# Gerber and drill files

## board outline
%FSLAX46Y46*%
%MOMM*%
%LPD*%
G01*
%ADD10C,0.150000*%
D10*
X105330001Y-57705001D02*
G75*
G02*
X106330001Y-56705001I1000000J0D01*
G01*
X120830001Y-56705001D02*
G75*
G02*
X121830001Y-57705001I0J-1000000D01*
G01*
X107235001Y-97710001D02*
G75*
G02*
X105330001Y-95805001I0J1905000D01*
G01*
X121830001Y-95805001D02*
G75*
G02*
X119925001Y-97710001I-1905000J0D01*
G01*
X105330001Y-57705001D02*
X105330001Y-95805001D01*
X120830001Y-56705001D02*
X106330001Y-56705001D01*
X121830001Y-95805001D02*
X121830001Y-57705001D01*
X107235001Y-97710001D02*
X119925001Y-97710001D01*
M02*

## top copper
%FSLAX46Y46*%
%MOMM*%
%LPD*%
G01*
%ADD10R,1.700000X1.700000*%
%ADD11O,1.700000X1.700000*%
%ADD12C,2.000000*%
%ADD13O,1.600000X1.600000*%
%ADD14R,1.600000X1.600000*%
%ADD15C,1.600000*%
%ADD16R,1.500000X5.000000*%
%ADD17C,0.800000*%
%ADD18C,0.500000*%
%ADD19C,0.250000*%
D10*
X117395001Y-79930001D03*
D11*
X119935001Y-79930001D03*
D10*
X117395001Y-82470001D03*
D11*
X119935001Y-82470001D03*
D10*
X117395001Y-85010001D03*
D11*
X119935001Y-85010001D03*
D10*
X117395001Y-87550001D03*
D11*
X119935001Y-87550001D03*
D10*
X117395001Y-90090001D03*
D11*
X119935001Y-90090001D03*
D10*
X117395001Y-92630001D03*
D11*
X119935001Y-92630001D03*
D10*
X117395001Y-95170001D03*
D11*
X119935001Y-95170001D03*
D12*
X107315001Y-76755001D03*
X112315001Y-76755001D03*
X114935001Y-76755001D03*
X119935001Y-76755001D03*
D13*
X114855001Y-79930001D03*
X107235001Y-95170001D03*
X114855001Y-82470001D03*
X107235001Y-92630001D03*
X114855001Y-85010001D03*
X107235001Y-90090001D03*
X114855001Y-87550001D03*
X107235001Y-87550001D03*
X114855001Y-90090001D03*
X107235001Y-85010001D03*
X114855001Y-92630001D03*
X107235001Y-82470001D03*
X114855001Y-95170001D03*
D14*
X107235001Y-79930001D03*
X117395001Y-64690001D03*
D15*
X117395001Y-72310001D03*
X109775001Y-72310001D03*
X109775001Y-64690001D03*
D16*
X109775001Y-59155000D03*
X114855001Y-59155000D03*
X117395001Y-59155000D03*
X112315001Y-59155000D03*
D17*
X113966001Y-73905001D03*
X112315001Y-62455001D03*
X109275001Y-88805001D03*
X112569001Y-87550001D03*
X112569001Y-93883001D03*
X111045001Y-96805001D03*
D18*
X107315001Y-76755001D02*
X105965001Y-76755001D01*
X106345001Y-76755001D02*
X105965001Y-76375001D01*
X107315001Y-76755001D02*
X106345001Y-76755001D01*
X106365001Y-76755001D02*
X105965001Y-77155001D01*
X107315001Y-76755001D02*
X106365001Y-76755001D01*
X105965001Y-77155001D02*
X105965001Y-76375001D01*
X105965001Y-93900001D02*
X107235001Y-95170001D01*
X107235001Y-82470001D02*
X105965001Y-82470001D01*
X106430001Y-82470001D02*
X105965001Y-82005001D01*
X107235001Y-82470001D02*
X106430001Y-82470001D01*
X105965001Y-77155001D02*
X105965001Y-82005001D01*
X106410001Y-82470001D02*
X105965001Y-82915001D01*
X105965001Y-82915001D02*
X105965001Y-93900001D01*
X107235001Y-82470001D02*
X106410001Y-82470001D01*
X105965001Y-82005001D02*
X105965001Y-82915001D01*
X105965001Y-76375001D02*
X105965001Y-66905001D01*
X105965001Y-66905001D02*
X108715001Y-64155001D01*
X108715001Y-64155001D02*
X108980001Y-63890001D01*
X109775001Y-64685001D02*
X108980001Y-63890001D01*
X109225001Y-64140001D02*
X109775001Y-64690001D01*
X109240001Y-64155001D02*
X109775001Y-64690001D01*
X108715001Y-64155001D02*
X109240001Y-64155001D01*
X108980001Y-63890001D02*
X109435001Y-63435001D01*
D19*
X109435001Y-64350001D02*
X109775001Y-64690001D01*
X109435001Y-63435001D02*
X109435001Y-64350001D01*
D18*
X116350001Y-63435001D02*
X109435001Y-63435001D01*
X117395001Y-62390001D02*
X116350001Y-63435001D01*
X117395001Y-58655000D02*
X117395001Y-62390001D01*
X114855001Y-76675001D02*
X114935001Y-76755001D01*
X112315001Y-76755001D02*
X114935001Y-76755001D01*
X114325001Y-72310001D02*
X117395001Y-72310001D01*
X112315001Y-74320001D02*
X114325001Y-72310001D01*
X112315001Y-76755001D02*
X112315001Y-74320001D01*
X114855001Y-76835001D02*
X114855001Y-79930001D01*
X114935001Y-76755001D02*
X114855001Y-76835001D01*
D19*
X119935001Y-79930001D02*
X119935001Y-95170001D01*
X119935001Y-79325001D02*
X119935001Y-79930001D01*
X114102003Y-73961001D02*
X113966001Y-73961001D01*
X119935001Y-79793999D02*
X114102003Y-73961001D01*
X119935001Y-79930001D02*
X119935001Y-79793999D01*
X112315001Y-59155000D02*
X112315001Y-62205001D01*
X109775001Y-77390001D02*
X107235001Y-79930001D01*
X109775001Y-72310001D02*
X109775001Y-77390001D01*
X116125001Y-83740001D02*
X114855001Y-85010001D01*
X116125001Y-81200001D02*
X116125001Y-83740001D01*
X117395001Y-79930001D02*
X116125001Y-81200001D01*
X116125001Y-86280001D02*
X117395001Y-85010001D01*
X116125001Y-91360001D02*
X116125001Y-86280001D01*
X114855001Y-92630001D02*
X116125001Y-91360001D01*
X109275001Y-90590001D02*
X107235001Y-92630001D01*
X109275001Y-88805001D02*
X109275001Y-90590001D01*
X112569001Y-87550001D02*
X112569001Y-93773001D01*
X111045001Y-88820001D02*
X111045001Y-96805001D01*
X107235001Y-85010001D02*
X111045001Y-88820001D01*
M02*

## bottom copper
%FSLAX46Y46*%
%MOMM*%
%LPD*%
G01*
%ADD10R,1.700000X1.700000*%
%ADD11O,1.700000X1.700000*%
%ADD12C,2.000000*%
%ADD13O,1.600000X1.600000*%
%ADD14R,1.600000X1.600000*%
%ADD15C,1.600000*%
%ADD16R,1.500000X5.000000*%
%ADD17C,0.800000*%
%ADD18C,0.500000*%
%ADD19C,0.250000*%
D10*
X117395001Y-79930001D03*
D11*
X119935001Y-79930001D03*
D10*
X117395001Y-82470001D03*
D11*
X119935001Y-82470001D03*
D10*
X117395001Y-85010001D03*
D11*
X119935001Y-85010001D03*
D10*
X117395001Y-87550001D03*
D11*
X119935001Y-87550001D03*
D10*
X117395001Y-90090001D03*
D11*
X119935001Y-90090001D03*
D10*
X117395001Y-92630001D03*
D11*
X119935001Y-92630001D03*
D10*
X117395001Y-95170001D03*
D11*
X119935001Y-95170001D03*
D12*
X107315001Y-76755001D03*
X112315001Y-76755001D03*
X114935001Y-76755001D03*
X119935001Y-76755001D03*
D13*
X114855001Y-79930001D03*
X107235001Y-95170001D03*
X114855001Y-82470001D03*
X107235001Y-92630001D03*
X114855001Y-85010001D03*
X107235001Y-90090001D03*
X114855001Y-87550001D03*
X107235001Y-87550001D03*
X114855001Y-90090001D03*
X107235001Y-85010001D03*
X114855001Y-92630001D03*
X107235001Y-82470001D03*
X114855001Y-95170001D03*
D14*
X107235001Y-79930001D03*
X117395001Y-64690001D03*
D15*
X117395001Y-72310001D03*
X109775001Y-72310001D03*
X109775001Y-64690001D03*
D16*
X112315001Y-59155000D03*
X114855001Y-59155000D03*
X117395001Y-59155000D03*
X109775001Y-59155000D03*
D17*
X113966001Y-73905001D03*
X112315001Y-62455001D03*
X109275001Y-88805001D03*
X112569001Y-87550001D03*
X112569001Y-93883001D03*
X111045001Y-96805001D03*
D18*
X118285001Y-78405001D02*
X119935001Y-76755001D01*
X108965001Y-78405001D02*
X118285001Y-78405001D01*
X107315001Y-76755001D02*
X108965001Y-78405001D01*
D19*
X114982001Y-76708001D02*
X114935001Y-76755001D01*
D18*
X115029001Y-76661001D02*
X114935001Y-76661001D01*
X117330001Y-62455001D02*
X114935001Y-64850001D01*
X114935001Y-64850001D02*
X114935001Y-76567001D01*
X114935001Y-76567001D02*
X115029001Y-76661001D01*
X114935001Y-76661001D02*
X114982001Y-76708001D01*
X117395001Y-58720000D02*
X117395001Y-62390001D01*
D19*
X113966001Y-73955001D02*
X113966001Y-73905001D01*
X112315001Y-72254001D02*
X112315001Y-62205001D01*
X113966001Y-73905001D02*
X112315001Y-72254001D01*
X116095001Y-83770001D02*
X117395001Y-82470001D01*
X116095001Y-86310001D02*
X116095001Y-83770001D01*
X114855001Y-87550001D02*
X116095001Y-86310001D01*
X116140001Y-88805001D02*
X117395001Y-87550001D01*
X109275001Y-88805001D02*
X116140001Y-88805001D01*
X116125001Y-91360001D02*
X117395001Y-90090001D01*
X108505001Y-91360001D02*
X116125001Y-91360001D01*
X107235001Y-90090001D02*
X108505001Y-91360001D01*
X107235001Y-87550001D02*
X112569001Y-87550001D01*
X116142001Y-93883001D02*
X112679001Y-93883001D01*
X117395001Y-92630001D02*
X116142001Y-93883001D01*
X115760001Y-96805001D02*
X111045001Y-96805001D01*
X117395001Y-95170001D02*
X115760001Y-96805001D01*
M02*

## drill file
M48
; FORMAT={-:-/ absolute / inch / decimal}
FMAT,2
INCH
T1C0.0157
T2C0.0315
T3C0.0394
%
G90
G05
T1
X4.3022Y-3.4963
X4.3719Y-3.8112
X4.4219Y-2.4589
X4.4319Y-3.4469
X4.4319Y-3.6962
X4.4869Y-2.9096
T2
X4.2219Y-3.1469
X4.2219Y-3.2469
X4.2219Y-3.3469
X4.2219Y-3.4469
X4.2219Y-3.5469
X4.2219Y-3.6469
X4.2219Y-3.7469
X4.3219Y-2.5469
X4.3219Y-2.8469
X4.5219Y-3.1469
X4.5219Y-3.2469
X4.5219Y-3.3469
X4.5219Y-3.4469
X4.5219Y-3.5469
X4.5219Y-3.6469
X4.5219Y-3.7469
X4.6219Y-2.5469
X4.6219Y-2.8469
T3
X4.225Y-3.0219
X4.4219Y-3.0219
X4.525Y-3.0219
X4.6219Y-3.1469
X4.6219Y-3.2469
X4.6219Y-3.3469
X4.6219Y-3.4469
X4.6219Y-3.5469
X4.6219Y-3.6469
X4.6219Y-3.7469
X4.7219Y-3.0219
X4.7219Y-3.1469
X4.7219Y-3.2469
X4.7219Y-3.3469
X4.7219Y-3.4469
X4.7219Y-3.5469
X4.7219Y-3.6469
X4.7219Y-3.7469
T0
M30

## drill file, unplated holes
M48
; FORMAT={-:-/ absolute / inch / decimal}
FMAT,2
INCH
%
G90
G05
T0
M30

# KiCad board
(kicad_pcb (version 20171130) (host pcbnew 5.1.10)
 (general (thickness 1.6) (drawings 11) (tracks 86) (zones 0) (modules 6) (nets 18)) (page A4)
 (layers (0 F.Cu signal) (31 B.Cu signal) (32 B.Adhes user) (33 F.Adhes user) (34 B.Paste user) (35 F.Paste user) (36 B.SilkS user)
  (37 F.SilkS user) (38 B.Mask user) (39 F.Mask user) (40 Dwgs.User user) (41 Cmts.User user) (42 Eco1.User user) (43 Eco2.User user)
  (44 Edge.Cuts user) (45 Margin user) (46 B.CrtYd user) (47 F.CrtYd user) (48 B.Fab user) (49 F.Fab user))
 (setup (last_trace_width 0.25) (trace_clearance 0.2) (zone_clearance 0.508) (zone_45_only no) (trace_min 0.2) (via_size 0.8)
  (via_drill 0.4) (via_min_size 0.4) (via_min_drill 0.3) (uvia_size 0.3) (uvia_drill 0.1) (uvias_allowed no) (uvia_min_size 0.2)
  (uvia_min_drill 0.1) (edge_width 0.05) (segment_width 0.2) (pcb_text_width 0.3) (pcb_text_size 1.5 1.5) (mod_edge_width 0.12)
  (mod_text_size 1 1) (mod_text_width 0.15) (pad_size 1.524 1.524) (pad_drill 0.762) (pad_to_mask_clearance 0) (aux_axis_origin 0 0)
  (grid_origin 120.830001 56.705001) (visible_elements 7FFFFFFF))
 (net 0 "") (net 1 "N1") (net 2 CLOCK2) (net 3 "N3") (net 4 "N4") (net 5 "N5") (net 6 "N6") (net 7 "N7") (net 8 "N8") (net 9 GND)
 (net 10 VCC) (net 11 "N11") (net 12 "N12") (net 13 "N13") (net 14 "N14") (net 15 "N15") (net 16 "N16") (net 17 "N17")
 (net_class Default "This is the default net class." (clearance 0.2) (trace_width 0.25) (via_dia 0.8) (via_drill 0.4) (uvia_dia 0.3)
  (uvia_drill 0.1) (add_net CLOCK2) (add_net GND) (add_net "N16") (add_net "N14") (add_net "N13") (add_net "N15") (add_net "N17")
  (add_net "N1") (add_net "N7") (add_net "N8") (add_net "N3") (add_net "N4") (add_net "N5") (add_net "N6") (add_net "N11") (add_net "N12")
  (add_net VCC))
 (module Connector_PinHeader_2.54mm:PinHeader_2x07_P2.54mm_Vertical (layer F.Cu) (at 117.395001 79.930001)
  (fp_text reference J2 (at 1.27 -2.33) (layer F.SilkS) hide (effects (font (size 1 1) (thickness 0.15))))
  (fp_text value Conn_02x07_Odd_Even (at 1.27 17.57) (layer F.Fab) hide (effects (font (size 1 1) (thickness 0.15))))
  (pad 1 thru_hole rect (at 0 0) (size 1.7 1.7) (drill 1) (layers *.Cu *.Mask) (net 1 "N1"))
  (pad 2 thru_hole oval (at 2.54 0) (size 1.7 1.7) (drill 1) (layers *.Cu *.Mask) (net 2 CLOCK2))
  (pad 3 thru_hole rect (at 0 2.54) (size 1.7 1.7) (drill 1) (layers *.Cu *.Mask) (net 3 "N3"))
  (pad 4 thru_hole oval (at 2.54 2.54) (size 1.7 1.7) (drill 1) (layers *.Cu *.Mask) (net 2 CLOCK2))
  (pad 5 thru_hole rect (at 0 5.08) (size 1.7 1.7) (drill 1) (layers *.Cu *.Mask) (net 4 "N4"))
  (pad 6 thru_hole oval (at 2.54 5.08) (size 1.7 1.7) (drill 1) (layers *.Cu *.Mask) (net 2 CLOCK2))
  (pad 7 thru_hole rect (at 0 7.62) (size 1.7 1.7) (drill 1) (layers *.Cu *.Mask) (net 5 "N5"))
  (pad 8 thru_hole oval (at 2.54 7.62) (size 1.7 1.7) (drill 1) (layers *.Cu *.Mask) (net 2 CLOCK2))
  (pad 9 thru_hole rect (at 0 10.16) (size 1.7 1.7) (drill 1) (layers *.Cu *.Mask) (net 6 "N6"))
  (pad 10 thru_hole oval (at 2.54 10.16) (size 1.7 1.7) (drill 1) (layers *.Cu *.Mask) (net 2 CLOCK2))
  (pad 11 thru_hole rect (at 0 12.7) (size 1.7 1.7) (drill 1) (layers *.Cu *.Mask) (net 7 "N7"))
  (pad 12 thru_hole oval (at 2.54 12.7) (size 1.7 1.7) (drill 1) (layers *.Cu *.Mask) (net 2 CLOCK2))
  (pad 13 thru_hole rect (at 0 15.24) (size 1.7 1.7) (drill 1) (layers *.Cu *.Mask) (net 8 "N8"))
  (pad 14 thru_hole oval (at 2.54 15.24) (size 1.7 1.7) (drill 1) (layers *.Cu *.Mask) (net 2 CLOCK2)))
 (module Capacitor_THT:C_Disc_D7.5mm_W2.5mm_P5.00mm (layer F.Cu) (at 112.315001 76.755001 180)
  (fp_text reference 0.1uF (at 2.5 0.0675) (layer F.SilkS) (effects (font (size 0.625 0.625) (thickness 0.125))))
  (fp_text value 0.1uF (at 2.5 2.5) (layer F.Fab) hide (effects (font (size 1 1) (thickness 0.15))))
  (pad 2 thru_hole circle (at 5 0 180) (size 2 2) (drill 1) (layers *.Cu *.Mask) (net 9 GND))
  (pad 1 thru_hole circle (at 0 0 180) (size 2 2) (drill 1) (layers *.Cu *.Mask) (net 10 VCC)))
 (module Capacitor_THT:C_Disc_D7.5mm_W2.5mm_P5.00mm (layer F.Cu) (at 114.935001 76.755001)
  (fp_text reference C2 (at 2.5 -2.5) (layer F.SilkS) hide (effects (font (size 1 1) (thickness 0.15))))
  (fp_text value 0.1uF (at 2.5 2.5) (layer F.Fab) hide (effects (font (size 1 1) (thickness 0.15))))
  (pad 1 thru_hole circle (at 0 0) (size 2 2) (drill 1) (layers *.Cu *.Mask) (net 10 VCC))
  (pad 2 thru_hole circle (at 5 0) (size 2 2) (drill 1) (layers *.Cu *.Mask) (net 9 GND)))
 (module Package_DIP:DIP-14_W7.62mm (layer F.Cu) (at 107.235001 79.930001)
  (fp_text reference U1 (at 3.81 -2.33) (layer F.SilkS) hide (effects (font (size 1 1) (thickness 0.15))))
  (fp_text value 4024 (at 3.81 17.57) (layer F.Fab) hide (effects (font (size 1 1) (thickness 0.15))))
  (pad 14 thru_hole oval (at 7.62 0) (size 1.6 1.6) (drill 0.8) (layers *.Cu *.Mask) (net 10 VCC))
  (pad 7 thru_hole oval (at 0 15.24) (size 1.6 1.6) (drill 0.8) (layers *.Cu *.Mask) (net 9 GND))
  (pad 13 thru_hole oval (at 7.62 2.54) (size 1.6 1.6) (drill 0.8) (layers *.Cu *.Mask))
  (pad 6 thru_hole oval (at 0 12.7) (size 1.6 1.6) (drill 0.8) (layers *.Cu *.Mask) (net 5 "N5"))
  (pad 12 thru_hole oval (at 7.62 5.08) (size 1.6 1.6) (drill 0.8) (layers *.Cu *.Mask) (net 1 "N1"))
  (pad 5 thru_hole oval (at 0 10.16) (size 1.6 1.6) (drill 0.8) (layers *.Cu *.Mask) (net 6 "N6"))
  (pad 11 thru_hole oval (at 7.62 7.62) (size 1.6 1.6) (drill 0.8) (layers *.Cu *.Mask) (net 3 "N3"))
  (pad 4 thru_hole oval (at 0 7.62) (size 1.6 1.6) (drill 0.8) (layers *.Cu *.Mask) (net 7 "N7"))
  (pad 10 thru_hole oval (at 7.62 10.16) (size 1.6 1.6) (drill 0.8) (layers *.Cu *.Mask))
  (pad 3 thru_hole oval (at 0 5.08) (size 1.6 1.6) (drill 0.8) (layers *.Cu *.Mask) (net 8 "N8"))
  (pad 9 thru_hole oval (at 7.62 12.7) (size 1.6 1.6) (drill 0.8) (layers *.Cu *.Mask) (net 4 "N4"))
  (pad 2 thru_hole oval (at 0 2.54) (size 1.6 1.6) (drill 0.8) (layers *.Cu *.Mask) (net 9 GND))
  (pad 8 thru_hole oval (at 7.62 15.24) (size 1.6 1.6) (drill 0.8) (layers *.Cu *.Mask))
  (pad 1 thru_hole rect (at 0 0) (size 1.6 1.6) (drill 0.8) (layers *.Cu *.Mask) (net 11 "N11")))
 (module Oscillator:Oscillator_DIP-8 (layer F.Cu) (at 117.395001 64.690001 180)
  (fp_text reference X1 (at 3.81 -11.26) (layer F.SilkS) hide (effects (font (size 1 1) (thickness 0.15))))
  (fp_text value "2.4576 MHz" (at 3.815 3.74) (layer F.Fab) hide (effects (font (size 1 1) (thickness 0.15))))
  (pad 1 thru_hole rect (at 0 0 180) (size 1.6 1.6) (drill 0.8) (layers *.Cu *.Mask) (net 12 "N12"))
  (pad 8 thru_hole circle (at 0 -7.62 180) (size 1.6 1.6) (drill 0.8) (layers *.Cu *.Mask) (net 10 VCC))
  (pad 5 thru_hole circle (at 7.62 -7.62 180) (size 1.6 1.6) (drill 0.8) (layers *.Cu *.Mask) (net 11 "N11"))
  (pad 4 thru_hole circle (at 7.62 0 180) (size 1.6 1.6) (drill 0.8) (layers *.Cu *.Mask) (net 9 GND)))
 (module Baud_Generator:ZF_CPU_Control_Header (layer F.Cu) (at 113.585001 59.028)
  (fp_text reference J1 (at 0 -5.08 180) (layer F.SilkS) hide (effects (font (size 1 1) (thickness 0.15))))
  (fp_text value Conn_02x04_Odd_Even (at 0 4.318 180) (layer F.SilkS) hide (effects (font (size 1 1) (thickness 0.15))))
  (pad 6 connect rect (at -1.27 0.127 180) (size 1.5 5) (layers B.Cu) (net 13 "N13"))
  (pad 4 connect rect (at 1.27 0.127 180) (size 1.5 5) (layers B.Cu) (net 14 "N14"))
  (pad 2 connect rect (at 3.81 0.127 180) (size 1.5 5) (layers B.Cu) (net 10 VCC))
  (pad 7 connect rect (at -3.81 0.127 180) (size 1.5 5) (layers F.Cu) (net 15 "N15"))
  (pad 3 connect rect (at 1.27 0.127 180) (size 1.5 5) (layers F.Cu) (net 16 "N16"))
  (pad 1 connect rect (at 3.81 0.127 180) (size 1.5 5) (layers F.Cu) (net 9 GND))
  (pad 5 connect rect (at -1.27 0.127 180) (size 1.5 5) (layers F.Cu) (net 2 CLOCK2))
  (pad 8 connect rect (at -3.81 0.127 180) (size 1.5 5) (layers B.Cu) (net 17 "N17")))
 (gr_arc (start 106.330001 57.705001) (end 106.330001 56.705001) (angle -90) (layer Edge.Cuts) (width 0.15))
 (gr_arc (start 120.830001 57.705001) (end 121.830001 57.705001) (angle -90) (layer Edge.Cuts) (width 0.15))
 (gr_arc (start 107.235001 95.805001) (end 105.330001 95.805001) (angle -90) (layer Edge.Cuts) (width 0.15))
 (gr_arc (start 119.925001 95.805001) (end 119.925001 97.710001) (angle -90) (layer Edge.Cuts) (width 0.15))
 (gr_line (start 105.330001 57.705001) (end 105.330001 95.805001) (layer Edge.Cuts) (width 0.15))
 (gr_line (start 120.830001 56.705001) (end 106.330001 56.705001) (layer Edge.Cuts) (width 0.15))
 (gr_line (start 121.830001 95.805001) (end 121.830001 57.705001) (layer Edge.Cuts) (width 0.15))
 (gr_line (start 107.235001 97.710001) (end 119.925001 97.710001) (layer Edge.Cuts) (width 0.15))
 (segment (start 107.315001 76.755001) (end 105.965001 76.755001) (width 0.5) (layer F.Cu) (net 9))
 (segment (start 106.345001 76.755001) (end 105.965001 76.375001) (width 0.5) (layer F.Cu) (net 9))
 (segment (start 107.315001 76.755001) (end 106.345001 76.755001) (width 0.5) (layer F.Cu) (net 9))
 (segment (start 106.365001 76.755001) (end 105.965001 77.155001) (width 0.5) (layer F.Cu) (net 9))
 (segment (start 107.315001 76.755001) (end 106.365001 76.755001) (width 0.5) (layer F.Cu) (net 9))
 (segment (start 105.965001 77.155001) (end 105.965001 76.375001) (width 0.5) (layer F.Cu) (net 9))
 (segment (start 105.965001 93.900001) (end 107.235001 95.170001) (width 0.5) (layer F.Cu) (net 9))
 (segment (start 107.235001 82.470001) (end 105.965001 82.470001) (width 0.5) (layer F.Cu) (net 9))
 (segment (start 106.430001 82.470001) (end 105.965001 82.005001) (width 0.5) (layer F.Cu) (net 9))
 (segment (start 107.235001 82.470001) (end 106.430001 82.470001) (width 0.5) (layer F.Cu) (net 9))
 (segment (start 105.965001 77.155001) (end 105.965001 82.005001) (width 0.5) (layer F.Cu) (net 9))
 (segment (start 106.410001 82.470001) (end 105.965001 82.915001) (width 0.5) (layer F.Cu) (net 9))
 (segment (start 105.965001 82.915001) (end 105.965001 93.900001) (width 0.5) (layer F.Cu) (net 9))
 (segment (start 107.235001 82.470001) (end 106.410001 82.470001) (width 0.5) (layer F.Cu) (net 9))
 (segment (start 105.965001 82.005001) (end 105.965001 82.915001) (width 0.5) (layer F.Cu) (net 9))
 (segment (start 105.965001 76.375001) (end 105.965001 66.905001) (width 0.5) (layer F.Cu) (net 9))
 (segment (start 105.965001 66.905001) (end 108.715001 64.155001) (width 0.5) (layer F.Cu) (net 9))
 (segment (start 108.715001 64.155001) (end 108.980001 63.890001) (width 0.5) (layer F.Cu) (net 9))
 (segment (start 109.775001 64.685001) (end 108.980001 63.890001) (width 0.5) (layer F.Cu) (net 9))
 (segment (start 109.225001 64.140001) (end 109.775001 64.690001) (width 0.5) (layer F.Cu) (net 9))
 (segment (start 109.240001 64.155001) (end 109.775001 64.690001) (width 0.5) (layer F.Cu) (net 9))
 (segment (start 108.715001 64.155001) (end 109.240001 64.155001) (width 0.5) (layer F.Cu) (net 9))
 (segment (start 118.285001 78.405001) (end 119.935001 76.755001) (width 0.5) (layer B.Cu) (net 9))
 (segment (start 108.965001 78.405001) (end 118.285001 78.405001) (width 0.5) (layer B.Cu) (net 9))
 (segment (start 107.315001 76.755001) (end 108.965001 78.405001) (width 0.5) (layer B.Cu) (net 9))
 (segment (start 108.980001 63.890001) (end 109.435001 63.435001) (width 0.5) (layer F.Cu) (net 9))
 (segment (start 109.435001 64.350001) (end 109.775001 64.690001) (width 0.25) (layer F.Cu) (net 9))
 (segment (start 109.435001 63.435001) (end 109.435001 64.350001) (width 0.25) (layer F.Cu) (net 9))
 (segment (start 116.350001 63.435001) (end 109.435001 63.435001) (width 0.5) (layer F.Cu) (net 9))
 (segment (start 117.395001 62.390001) (end 116.350001 63.435001) (width 0.5) (layer F.Cu) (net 9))
 (segment (start 117.395001 58.655) (end 117.395001 62.390001) (width 0.5) (layer F.Cu) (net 9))
 (segment (start 114.855001 76.675001) (end 114.935001 76.755001) (width 0.5) (layer F.Cu) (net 10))
 (segment (start 112.315001 76.755001) (end 114.935001 76.755001) (width 0.5) (layer F.Cu) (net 10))
 (segment (start 114.982001 76.708001) (end 114.935001 76.755001) (width 0.25) (layer B.Cu) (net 10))
 (segment (start 114.325001 72.310001) (end 117.395001 72.310001) (width 0.5) (layer F.Cu) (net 10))
 (segment (start 112.315001 74.320001) (end 114.325001 72.310001) (width 0.5) (layer F.Cu) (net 10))
 (segment (start 112.315001 76.755001) (end 112.315001 74.320001) (width 0.5) (layer F.Cu) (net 10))
 (segment (start 114.855001 76.835001) (end 114.855001 79.930001) (width 0.5) (layer F.Cu) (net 10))
 (segment (start 114.935001 76.755001) (end 114.855001 76.835001) (width 0.5) (layer F.Cu) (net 10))
 (segment (start 115.029001 76.661001) (end 114.935001 76.661001) (width 0.5) (layer B.Cu) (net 10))
 (segment (start 117.330001 62.455001) (end 114.935001 64.850001) (width 0.5) (layer B.Cu) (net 10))
 (segment (start 114.935001 64.850001) (end 114.935001 76.567001) (width 0.5) (layer B.Cu) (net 10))
 (segment (start 114.935001 76.567001) (end 115.029001 76.661001) (width 0.5) (layer B.Cu) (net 10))
 (segment (start 114.935001 76.661001) (end 114.982001 76.708001) (width 0.5) (layer B.Cu) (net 10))
 (segment (start 117.395001 58.72) (end 117.395001 62.390001) (width 0.5) (layer B.Cu) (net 10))
 (segment (start 119.935001 79.930001) (end 119.935001 95.170001) (width 0.25) (layer F.Cu) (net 2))
 (segment (start 119.935001 79.325001) (end 119.935001 79.930001) (width 0.25) (layer F.Cu) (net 2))
 (via (at 113.966001 73.905001) (size 0.8) (drill 0.4) (layers F.Cu B.Cu) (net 2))
 (via (at 112.315001 62.455001) (size 0.8) (drill 0.4) (layers F.Cu B.Cu) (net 2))
 (segment (start 114.102003 73.961001) (end 113.966001 73.961001) (width 0.25) (layer F.Cu) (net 2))
 (segment (start 119.935001 79.793999) (end 114.102003 73.961001) (width 0.25) (layer F.Cu) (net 2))
 (segment (start 119.935001 79.930001) (end 119.935001 79.793999) (width 0.25) (layer F.Cu) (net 2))
 (segment (start 113.966001 73.955001) (end 113.966001 73.905001) (width 0.25) (layer B.Cu) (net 2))
 (segment (start 112.315001 59.155) (end 112.315001 62.205001) (width 0.25) (layer F.Cu) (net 2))
 (segment (start 112.315001 72.254001) (end 112.315001 62.205001) (width 0.25) (layer B.Cu) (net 2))
 (segment (start 113.966001 73.905001) (end 112.315001 72.254001) (width 0.25) (layer B.Cu) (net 2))
 (segment (start 109.775001 77.390001) (end 107.235001 79.930001) (width 0.25) (layer F.Cu) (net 11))
 (segment (start 109.775001 72.310001) (end 109.775001 77.390001) (width 0.25) (layer F.Cu) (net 11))
 (segment (start 116.125001 83.740001) (end 114.855001 85.010001) (width 0.25) (layer F.Cu) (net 1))
 (segment (start 116.125001 81.200001) (end 116.125001 83.740001) (width 0.25) (layer F.Cu) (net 1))
 (segment (start 117.395001 79.930001) (end 116.125001 81.200001) (width 0.25) (layer F.Cu) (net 1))
 (segment (start 116.095001 83.770001) (end 117.395001 82.470001) (width 0.25) (layer B.Cu) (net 3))
 (segment (start 116.095001 86.310001) (end 116.095001 83.770001) (width 0.25) (layer B.Cu) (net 3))
 (segment (start 114.855001 87.550001) (end 116.095001 86.310001) (width 0.25) (layer B.Cu) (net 3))
 (segment (start 116.125001 86.280001) (end 117.395001 85.010001) (width 0.25) (layer F.Cu) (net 4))
 (segment (start 116.125001 91.360001) (end 116.125001 86.280001) (width 0.25) (layer F.Cu) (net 4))
 (segment (start 114.855001 92.630001) (end 116.125001 91.360001) (width 0.25) (layer F.Cu) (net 4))
 (via (at 109.275001 88.805001) (size 0.8) (drill 0.4) (layers F.Cu B.Cu) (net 5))
 (segment (start 116.140001 88.805001) (end 117.395001 87.550001) (width 0.25) (layer B.Cu) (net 5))
 (segment (start 109.275001 88.805001) (end 116.140001 88.805001) (width 0.25) (layer B.Cu) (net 5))
 (segment (start 109.275001 90.590001) (end 107.235001 92.630001) (width 0.25) (layer F.Cu) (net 5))
 (segment (start 109.275001 88.805001) (end 109.275001 90.590001) (width 0.25) (layer F.Cu) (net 5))
 (segment (start 116.125001 91.360001) (end 117.395001 90.090001) (width 0.25) (layer B.Cu) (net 6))
 (segment (start 108.505001 91.360001) (end 116.125001 91.360001) (width 0.25) (layer B.Cu) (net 6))
 (segment (start 107.235001 90.090001) (end 108.505001 91.360001) (width 0.25) (layer B.Cu) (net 6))
 (via (at 112.569001 87.550001) (size 0.8) (drill 0.4) (layers F.Cu B.Cu) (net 7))
 (via (at 112.569001 93.883001) (size 0.8) (drill 0.4) (layers F.Cu B.Cu) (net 7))
 (segment (start 112.569001 87.550001) (end 112.569001 93.773001) (width 0.25) (layer F.Cu) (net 7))
 (segment (start 107.235001 87.550001) (end 112.569001 87.550001) (width 0.25) (layer B.Cu) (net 7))
 (segment (start 116.142001 93.883001) (end 112.679001 93.883001) (width 0.25) (layer B.Cu) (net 7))
 (segment (start 117.395001 92.630001) (end 116.142001 93.883001) (width 0.25) (layer B.Cu) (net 7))
 (via (at 111.045001 96.805001) (size 0.8) (drill 0.4) (layers F.Cu B.Cu) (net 8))
 (segment (start 111.045001 88.820001) (end 111.045001 96.805001) (width 0.25) (layer F.Cu) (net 8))
 (segment (start 107.235001 85.010001) (end 111.045001 88.820001) (width 0.25) (layer F.Cu) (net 8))
 (segment (start 115.760001 96.805001) (end 111.045001 96.805001) (width 0.25) (layer B.Cu) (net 8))
 (segment (start 117.395001 95.170001) (end 115.760001 96.805001) (width 0.25) (layer B.Cu) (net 8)))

